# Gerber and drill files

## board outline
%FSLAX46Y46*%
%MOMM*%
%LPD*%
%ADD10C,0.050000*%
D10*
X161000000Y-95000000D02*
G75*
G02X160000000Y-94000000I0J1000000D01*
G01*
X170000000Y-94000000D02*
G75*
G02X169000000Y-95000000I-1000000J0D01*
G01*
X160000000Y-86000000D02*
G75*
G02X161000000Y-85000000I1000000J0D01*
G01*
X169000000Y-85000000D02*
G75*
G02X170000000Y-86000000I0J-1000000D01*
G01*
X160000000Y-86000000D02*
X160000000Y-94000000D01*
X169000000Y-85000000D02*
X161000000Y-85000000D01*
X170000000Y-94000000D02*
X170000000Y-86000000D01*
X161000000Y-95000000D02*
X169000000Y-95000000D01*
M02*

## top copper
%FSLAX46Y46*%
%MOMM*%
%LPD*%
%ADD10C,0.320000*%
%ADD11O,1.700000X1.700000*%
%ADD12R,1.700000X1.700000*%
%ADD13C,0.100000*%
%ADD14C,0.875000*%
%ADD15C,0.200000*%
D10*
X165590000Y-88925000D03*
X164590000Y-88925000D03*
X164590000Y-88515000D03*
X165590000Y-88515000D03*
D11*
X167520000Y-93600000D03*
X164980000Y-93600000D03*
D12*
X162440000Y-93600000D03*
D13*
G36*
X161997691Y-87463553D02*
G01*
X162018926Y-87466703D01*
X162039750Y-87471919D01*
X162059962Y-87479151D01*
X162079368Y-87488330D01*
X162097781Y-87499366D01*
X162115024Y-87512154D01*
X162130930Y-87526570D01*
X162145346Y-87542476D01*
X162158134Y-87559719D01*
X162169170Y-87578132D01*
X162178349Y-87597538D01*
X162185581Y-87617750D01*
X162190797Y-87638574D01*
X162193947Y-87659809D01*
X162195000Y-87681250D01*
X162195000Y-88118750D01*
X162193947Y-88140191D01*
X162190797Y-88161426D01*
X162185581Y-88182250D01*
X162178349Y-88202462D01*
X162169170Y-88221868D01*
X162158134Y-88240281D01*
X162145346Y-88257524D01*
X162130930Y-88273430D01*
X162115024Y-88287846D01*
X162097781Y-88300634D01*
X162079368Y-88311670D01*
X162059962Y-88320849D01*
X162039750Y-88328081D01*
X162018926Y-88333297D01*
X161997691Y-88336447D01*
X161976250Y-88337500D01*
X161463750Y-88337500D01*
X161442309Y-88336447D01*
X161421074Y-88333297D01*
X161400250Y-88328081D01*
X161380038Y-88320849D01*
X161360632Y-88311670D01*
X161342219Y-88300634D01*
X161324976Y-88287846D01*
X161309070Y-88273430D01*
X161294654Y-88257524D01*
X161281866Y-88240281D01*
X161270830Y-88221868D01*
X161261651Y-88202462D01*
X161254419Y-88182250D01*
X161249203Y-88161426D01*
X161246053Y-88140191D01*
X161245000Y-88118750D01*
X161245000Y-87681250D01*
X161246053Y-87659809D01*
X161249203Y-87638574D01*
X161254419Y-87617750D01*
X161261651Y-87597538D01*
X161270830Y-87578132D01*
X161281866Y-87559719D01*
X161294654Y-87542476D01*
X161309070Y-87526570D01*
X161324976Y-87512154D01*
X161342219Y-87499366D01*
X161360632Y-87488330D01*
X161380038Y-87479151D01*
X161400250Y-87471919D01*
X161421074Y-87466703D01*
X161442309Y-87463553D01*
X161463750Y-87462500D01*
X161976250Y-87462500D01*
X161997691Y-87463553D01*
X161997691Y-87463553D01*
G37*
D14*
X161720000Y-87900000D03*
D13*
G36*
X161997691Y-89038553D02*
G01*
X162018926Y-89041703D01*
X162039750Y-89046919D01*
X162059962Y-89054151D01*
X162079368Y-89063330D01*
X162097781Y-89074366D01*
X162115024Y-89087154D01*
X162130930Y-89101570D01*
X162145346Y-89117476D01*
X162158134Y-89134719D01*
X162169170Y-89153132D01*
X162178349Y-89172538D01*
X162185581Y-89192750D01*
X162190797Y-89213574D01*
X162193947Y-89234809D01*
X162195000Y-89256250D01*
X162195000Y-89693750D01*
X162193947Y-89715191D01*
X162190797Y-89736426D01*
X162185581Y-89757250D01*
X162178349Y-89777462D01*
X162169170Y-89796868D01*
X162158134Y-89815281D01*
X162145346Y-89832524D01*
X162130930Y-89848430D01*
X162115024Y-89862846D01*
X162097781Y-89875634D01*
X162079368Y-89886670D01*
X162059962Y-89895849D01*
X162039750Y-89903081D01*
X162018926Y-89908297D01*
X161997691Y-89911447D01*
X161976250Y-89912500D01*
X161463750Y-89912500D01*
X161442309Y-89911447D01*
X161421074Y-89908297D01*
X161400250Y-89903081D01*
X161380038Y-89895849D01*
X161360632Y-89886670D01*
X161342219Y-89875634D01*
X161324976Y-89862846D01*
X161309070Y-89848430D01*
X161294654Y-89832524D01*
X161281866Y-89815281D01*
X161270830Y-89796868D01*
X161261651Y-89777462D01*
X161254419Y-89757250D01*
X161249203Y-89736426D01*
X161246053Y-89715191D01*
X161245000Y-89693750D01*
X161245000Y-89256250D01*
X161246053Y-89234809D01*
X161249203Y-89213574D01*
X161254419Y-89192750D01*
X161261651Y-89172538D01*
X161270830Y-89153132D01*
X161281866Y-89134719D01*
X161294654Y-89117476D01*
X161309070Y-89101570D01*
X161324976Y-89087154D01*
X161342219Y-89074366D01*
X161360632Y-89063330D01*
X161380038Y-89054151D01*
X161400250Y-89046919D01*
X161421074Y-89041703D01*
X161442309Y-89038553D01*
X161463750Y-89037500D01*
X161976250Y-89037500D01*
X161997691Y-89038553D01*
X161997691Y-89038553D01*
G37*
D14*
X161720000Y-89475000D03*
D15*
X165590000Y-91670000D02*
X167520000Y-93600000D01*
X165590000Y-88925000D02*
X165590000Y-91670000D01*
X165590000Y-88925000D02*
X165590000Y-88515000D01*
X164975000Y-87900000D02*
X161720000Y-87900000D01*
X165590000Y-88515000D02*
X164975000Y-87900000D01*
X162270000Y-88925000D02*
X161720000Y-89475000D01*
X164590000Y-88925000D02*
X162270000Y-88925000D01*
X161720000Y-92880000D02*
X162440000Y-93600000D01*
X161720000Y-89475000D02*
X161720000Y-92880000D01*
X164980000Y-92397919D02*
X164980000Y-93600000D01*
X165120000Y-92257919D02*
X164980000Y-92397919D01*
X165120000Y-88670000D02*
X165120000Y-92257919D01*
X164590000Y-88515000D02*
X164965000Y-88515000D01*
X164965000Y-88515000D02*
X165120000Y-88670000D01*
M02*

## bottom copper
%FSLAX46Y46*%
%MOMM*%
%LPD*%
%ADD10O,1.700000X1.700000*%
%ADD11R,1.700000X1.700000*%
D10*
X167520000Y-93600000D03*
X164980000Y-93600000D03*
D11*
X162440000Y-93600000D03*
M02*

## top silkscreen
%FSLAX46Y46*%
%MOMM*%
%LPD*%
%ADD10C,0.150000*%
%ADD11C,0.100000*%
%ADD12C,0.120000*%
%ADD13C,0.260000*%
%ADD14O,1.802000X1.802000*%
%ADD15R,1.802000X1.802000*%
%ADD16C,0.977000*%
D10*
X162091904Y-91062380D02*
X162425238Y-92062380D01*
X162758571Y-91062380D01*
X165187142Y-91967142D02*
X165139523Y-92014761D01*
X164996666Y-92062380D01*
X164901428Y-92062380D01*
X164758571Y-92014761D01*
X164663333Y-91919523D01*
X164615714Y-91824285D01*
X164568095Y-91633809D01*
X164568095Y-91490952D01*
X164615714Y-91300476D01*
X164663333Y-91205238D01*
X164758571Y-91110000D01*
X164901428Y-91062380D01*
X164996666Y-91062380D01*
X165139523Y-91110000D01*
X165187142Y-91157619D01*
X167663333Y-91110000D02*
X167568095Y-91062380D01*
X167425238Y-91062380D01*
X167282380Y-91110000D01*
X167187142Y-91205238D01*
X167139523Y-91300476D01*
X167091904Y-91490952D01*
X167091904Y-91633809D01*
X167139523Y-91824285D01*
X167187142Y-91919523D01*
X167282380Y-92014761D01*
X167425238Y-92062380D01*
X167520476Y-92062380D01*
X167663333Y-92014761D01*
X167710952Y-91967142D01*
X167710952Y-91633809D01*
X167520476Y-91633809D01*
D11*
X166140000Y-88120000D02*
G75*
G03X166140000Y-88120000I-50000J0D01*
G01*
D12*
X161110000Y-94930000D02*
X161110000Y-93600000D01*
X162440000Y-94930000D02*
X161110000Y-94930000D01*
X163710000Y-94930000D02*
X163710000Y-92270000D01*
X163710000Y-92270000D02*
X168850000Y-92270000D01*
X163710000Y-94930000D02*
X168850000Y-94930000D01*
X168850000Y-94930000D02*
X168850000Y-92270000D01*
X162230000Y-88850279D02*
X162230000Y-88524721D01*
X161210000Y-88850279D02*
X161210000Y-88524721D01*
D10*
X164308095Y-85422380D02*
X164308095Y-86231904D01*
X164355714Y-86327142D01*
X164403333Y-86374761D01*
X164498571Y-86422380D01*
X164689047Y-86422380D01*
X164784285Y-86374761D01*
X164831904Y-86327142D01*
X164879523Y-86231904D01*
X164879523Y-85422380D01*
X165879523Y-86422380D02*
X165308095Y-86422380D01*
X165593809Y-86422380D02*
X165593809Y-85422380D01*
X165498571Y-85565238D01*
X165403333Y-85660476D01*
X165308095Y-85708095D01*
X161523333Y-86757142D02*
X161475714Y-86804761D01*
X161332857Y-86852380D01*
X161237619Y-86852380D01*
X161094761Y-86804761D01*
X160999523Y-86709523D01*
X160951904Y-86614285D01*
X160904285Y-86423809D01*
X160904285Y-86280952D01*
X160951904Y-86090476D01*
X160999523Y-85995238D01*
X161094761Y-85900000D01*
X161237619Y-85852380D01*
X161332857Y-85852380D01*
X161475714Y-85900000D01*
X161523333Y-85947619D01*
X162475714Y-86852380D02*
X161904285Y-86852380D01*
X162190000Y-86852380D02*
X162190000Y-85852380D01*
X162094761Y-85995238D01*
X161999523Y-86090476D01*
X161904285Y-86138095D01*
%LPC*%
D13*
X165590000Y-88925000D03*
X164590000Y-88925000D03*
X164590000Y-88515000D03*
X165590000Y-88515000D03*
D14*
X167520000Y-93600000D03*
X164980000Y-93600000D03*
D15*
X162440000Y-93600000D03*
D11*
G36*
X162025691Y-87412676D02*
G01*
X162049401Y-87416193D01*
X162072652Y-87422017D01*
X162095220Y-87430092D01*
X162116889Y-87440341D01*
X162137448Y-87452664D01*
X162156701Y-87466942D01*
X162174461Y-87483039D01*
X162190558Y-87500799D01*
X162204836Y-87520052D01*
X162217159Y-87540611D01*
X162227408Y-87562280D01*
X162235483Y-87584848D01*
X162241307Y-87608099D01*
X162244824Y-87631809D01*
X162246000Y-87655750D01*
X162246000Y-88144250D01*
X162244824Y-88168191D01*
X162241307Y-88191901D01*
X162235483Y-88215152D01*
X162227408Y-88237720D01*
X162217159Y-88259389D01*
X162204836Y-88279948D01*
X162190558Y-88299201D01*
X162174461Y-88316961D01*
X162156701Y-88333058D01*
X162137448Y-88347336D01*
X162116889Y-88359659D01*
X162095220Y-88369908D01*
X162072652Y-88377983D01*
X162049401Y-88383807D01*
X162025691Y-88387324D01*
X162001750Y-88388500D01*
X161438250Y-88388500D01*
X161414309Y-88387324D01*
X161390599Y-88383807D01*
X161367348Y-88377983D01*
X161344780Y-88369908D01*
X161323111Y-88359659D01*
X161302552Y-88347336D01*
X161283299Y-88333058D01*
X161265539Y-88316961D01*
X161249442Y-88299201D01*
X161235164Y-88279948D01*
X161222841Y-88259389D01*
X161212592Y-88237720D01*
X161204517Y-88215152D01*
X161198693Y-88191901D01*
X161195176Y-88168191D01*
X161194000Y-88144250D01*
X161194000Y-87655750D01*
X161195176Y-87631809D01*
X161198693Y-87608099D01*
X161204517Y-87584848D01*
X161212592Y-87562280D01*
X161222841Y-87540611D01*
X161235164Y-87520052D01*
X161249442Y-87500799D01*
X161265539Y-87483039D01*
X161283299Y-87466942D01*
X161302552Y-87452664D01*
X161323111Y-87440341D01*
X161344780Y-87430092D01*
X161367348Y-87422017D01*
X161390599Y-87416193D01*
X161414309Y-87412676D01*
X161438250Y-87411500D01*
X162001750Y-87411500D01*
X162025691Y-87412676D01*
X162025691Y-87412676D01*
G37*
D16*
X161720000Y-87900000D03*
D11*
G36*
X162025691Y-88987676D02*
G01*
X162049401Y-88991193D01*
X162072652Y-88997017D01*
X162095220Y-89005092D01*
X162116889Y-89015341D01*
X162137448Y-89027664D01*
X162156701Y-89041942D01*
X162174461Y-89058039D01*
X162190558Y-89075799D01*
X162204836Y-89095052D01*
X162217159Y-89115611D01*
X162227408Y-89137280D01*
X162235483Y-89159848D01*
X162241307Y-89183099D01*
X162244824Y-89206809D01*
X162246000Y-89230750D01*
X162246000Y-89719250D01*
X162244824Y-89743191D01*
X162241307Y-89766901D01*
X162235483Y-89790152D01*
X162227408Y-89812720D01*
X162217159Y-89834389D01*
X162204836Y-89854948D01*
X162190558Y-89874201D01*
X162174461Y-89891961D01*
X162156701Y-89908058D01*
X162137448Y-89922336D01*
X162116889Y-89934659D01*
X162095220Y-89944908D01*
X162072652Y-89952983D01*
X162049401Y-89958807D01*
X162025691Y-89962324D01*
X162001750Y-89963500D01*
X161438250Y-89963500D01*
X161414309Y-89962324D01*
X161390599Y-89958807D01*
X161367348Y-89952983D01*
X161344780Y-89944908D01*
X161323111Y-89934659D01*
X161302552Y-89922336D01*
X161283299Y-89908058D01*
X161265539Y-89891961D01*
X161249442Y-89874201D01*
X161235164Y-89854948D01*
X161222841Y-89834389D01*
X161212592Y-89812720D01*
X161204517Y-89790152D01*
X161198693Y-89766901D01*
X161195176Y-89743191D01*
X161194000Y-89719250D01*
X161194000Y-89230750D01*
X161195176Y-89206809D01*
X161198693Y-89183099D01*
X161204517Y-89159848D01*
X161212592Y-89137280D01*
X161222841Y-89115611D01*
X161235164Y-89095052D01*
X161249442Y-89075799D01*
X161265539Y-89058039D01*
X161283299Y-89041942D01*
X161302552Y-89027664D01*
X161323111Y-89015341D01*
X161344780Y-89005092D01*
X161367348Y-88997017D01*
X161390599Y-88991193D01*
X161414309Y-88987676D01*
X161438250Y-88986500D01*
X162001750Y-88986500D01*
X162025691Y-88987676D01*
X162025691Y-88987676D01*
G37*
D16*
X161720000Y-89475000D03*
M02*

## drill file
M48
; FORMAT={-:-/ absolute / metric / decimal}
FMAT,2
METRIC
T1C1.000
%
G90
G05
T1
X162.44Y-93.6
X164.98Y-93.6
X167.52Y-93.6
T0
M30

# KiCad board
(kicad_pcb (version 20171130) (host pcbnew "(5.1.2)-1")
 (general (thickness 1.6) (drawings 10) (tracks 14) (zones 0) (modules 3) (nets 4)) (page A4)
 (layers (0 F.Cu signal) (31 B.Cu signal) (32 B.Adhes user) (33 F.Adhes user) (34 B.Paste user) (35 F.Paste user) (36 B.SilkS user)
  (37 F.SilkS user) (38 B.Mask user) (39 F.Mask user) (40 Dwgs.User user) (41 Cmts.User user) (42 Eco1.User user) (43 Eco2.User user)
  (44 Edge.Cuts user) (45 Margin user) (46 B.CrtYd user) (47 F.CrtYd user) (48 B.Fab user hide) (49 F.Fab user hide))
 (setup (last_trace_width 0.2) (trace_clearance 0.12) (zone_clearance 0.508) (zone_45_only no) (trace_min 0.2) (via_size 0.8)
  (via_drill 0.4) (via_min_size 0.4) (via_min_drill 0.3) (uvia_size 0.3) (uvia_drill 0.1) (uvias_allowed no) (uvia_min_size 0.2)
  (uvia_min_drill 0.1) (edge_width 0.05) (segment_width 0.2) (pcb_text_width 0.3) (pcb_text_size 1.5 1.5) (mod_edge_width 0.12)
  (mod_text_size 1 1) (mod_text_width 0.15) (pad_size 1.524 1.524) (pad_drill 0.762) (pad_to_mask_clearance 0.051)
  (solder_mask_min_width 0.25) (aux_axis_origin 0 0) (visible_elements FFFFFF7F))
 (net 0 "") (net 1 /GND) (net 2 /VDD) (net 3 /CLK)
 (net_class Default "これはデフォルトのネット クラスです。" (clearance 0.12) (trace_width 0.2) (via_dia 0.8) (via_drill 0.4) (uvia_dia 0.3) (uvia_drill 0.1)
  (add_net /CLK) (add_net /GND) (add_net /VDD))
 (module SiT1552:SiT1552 (layer F.Cu) (at 165.09 88.72 180)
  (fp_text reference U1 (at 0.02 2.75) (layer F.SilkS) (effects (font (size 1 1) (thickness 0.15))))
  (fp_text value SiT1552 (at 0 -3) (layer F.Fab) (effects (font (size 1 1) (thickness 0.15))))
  (fp_circle (center -1 0.6) (end -0.95 0.6) (layer F.SilkS) (width 0.1))
  (pad 4 smd circle (at -0.5 -0.205 180) (size 0.32 0.32) (layers F.Cu F.Paste F.Mask) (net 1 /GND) (solder_mask_margin -0.03)
   (solder_paste_margin -0.03))
  (pad 3 smd circle (at 0.5 -0.205 180) (size 0.32 0.32) (layers F.Cu F.Paste F.Mask) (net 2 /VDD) (solder_mask_margin -0.03)
   (solder_paste_margin -0.03))
  (pad 2 smd circle (at 0.5 0.205 180) (size 0.32 0.32) (layers F.Cu F.Paste F.Mask) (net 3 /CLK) (solder_mask_margin -0.03)
   (solder_paste_margin -0.03))
  (pad 1 smd circle (at -0.5 0.205 180) (size 0.32 0.32) (layers F.Cu F.Paste F.Mask) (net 1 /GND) (solder_mask_margin -0.03)
   (solder_paste_margin -0.03)))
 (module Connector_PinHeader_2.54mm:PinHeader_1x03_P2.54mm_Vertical (layer F.Cu) (at 162.44 93.6 90)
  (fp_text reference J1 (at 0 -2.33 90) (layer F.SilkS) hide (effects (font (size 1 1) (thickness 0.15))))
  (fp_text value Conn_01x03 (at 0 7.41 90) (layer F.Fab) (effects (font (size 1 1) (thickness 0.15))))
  (fp_line (start -1.33 -1.33) (end 0 -1.33) (layer F.SilkS) (width 0.12))
  (fp_line (start -1.33 0) (end -1.33 -1.33) (layer F.SilkS) (width 0.12))
  (fp_line (start -1.33 1.27) (end 1.33 1.27) (layer F.SilkS) (width 0.12))
  (fp_line (start 1.33 1.27) (end 1.33 6.41) (layer F.SilkS) (width 0.12))
  (fp_line (start -1.33 1.27) (end -1.33 6.41) (layer F.SilkS) (width 0.12))
  (fp_line (start -1.33 6.41) (end 1.33 6.41) (layer F.SilkS) (width 0.12))
  (pad 3 thru_hole oval (at 0 5.08 90) (size 1.7 1.7) (drill 1) (layers *.Cu *.Mask) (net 1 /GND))
  (pad 2 thru_hole oval (at 0 2.54 90) (size 1.7 1.7) (drill 1) (layers *.Cu *.Mask) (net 3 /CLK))
  (pad 1 thru_hole rect (at 0 0 90) (size 1.7 1.7) (drill 1) (layers *.Cu *.Mask) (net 2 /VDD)))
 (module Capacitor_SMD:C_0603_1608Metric (layer F.Cu) (at 161.72 88.6875 90)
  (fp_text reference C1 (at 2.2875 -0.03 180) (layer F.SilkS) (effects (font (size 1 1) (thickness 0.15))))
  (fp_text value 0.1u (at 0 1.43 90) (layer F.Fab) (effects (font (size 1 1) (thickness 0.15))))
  (fp_line (start -0.162779 0.51) (end 0.162779 0.51) (layer F.SilkS) (width 0.12))
  (fp_line (start -0.162779 -0.51) (end 0.162779 -0.51) (layer F.SilkS) (width 0.12))
  (pad 2 smd roundrect (at 0.7875 0 90) (size 0.875 0.95) (layers F.Cu F.Paste F.Mask) (roundrect_rratio 0.25) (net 1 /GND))
  (pad 1 smd roundrect (at -0.7875 0 90) (size 0.875 0.95) (layers F.Cu F.Paste F.Mask) (roundrect_rratio 0.25) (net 2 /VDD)))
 (gr_arc (start 161 94) (end 160 94) (angle -90) (layer Edge.Cuts) (width 0.05))
 (gr_arc (start 169 94) (end 169 95) (angle -90) (layer Edge.Cuts) (width 0.05))
 (gr_arc (start 161 86) (end 161 85) (angle -90) (layer Edge.Cuts) (width 0.05))
 (gr_arc (start 169 86) (end 170 86) (angle -90) (layer Edge.Cuts) (width 0.05))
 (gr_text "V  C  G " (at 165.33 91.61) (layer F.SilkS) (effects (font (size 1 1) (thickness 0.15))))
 (gr_line (start 160 86) (end 160 94) (layer Edge.Cuts) (width 0.05))
 (gr_line (start 169 85) (end 161 85) (layer Edge.Cuts) (width 0.05))
 (gr_line (start 170 94) (end 170 86) (layer Edge.Cuts) (width 0.05))
 (gr_line (start 161 95) (end 169 95) (layer Edge.Cuts) (width 0.05))
 (segment (start 165.59 91.67) (end 167.52 93.6) (width 0.2) (layer F.Cu) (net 1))
 (segment (start 165.59 88.925) (end 165.59 91.67) (width 0.2) (layer F.Cu) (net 1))
 (segment (start 165.59 88.925) (end 165.59 88.515) (width 0.2) (layer F.Cu) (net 1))
 (segment (start 164.975 87.9) (end 161.72 87.9) (width 0.2) (layer F.Cu) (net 1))
 (segment (start 165.59 88.515) (end 164.975 87.9) (width 0.2) (layer F.Cu) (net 1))
 (segment (start 162.27 88.925) (end 161.72 89.475) (width 0.2) (layer F.Cu) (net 2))
 (segment (start 164.59 88.925) (end 162.27 88.925) (width 0.2) (layer F.Cu) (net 2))
 (segment (start 161.72 92.88) (end 162.44 93.6) (width 0.2) (layer F.Cu) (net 2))
 (segment (start 161.72 89.475) (end 161.72 92.88) (width 0.2) (layer F.Cu) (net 2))
 (segment (start 164.98 92.397919) (end 164.98 93.6) (width 0.2) (layer F.Cu) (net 3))
 (segment (start 165.12 92.257919) (end 164.98 92.397919) (width 0.2) (layer F.Cu) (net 3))
 (segment (start 165.12 88.67) (end 165.12 92.257919) (width 0.2) (layer F.Cu) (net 3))
 (segment (start 164.59 88.515) (end 164.965 88.515) (width 0.2) (layer F.Cu) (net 3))
 (segment (start 164.965 88.515) (end 165.12 88.67) (width 0.2) (layer F.Cu) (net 3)))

